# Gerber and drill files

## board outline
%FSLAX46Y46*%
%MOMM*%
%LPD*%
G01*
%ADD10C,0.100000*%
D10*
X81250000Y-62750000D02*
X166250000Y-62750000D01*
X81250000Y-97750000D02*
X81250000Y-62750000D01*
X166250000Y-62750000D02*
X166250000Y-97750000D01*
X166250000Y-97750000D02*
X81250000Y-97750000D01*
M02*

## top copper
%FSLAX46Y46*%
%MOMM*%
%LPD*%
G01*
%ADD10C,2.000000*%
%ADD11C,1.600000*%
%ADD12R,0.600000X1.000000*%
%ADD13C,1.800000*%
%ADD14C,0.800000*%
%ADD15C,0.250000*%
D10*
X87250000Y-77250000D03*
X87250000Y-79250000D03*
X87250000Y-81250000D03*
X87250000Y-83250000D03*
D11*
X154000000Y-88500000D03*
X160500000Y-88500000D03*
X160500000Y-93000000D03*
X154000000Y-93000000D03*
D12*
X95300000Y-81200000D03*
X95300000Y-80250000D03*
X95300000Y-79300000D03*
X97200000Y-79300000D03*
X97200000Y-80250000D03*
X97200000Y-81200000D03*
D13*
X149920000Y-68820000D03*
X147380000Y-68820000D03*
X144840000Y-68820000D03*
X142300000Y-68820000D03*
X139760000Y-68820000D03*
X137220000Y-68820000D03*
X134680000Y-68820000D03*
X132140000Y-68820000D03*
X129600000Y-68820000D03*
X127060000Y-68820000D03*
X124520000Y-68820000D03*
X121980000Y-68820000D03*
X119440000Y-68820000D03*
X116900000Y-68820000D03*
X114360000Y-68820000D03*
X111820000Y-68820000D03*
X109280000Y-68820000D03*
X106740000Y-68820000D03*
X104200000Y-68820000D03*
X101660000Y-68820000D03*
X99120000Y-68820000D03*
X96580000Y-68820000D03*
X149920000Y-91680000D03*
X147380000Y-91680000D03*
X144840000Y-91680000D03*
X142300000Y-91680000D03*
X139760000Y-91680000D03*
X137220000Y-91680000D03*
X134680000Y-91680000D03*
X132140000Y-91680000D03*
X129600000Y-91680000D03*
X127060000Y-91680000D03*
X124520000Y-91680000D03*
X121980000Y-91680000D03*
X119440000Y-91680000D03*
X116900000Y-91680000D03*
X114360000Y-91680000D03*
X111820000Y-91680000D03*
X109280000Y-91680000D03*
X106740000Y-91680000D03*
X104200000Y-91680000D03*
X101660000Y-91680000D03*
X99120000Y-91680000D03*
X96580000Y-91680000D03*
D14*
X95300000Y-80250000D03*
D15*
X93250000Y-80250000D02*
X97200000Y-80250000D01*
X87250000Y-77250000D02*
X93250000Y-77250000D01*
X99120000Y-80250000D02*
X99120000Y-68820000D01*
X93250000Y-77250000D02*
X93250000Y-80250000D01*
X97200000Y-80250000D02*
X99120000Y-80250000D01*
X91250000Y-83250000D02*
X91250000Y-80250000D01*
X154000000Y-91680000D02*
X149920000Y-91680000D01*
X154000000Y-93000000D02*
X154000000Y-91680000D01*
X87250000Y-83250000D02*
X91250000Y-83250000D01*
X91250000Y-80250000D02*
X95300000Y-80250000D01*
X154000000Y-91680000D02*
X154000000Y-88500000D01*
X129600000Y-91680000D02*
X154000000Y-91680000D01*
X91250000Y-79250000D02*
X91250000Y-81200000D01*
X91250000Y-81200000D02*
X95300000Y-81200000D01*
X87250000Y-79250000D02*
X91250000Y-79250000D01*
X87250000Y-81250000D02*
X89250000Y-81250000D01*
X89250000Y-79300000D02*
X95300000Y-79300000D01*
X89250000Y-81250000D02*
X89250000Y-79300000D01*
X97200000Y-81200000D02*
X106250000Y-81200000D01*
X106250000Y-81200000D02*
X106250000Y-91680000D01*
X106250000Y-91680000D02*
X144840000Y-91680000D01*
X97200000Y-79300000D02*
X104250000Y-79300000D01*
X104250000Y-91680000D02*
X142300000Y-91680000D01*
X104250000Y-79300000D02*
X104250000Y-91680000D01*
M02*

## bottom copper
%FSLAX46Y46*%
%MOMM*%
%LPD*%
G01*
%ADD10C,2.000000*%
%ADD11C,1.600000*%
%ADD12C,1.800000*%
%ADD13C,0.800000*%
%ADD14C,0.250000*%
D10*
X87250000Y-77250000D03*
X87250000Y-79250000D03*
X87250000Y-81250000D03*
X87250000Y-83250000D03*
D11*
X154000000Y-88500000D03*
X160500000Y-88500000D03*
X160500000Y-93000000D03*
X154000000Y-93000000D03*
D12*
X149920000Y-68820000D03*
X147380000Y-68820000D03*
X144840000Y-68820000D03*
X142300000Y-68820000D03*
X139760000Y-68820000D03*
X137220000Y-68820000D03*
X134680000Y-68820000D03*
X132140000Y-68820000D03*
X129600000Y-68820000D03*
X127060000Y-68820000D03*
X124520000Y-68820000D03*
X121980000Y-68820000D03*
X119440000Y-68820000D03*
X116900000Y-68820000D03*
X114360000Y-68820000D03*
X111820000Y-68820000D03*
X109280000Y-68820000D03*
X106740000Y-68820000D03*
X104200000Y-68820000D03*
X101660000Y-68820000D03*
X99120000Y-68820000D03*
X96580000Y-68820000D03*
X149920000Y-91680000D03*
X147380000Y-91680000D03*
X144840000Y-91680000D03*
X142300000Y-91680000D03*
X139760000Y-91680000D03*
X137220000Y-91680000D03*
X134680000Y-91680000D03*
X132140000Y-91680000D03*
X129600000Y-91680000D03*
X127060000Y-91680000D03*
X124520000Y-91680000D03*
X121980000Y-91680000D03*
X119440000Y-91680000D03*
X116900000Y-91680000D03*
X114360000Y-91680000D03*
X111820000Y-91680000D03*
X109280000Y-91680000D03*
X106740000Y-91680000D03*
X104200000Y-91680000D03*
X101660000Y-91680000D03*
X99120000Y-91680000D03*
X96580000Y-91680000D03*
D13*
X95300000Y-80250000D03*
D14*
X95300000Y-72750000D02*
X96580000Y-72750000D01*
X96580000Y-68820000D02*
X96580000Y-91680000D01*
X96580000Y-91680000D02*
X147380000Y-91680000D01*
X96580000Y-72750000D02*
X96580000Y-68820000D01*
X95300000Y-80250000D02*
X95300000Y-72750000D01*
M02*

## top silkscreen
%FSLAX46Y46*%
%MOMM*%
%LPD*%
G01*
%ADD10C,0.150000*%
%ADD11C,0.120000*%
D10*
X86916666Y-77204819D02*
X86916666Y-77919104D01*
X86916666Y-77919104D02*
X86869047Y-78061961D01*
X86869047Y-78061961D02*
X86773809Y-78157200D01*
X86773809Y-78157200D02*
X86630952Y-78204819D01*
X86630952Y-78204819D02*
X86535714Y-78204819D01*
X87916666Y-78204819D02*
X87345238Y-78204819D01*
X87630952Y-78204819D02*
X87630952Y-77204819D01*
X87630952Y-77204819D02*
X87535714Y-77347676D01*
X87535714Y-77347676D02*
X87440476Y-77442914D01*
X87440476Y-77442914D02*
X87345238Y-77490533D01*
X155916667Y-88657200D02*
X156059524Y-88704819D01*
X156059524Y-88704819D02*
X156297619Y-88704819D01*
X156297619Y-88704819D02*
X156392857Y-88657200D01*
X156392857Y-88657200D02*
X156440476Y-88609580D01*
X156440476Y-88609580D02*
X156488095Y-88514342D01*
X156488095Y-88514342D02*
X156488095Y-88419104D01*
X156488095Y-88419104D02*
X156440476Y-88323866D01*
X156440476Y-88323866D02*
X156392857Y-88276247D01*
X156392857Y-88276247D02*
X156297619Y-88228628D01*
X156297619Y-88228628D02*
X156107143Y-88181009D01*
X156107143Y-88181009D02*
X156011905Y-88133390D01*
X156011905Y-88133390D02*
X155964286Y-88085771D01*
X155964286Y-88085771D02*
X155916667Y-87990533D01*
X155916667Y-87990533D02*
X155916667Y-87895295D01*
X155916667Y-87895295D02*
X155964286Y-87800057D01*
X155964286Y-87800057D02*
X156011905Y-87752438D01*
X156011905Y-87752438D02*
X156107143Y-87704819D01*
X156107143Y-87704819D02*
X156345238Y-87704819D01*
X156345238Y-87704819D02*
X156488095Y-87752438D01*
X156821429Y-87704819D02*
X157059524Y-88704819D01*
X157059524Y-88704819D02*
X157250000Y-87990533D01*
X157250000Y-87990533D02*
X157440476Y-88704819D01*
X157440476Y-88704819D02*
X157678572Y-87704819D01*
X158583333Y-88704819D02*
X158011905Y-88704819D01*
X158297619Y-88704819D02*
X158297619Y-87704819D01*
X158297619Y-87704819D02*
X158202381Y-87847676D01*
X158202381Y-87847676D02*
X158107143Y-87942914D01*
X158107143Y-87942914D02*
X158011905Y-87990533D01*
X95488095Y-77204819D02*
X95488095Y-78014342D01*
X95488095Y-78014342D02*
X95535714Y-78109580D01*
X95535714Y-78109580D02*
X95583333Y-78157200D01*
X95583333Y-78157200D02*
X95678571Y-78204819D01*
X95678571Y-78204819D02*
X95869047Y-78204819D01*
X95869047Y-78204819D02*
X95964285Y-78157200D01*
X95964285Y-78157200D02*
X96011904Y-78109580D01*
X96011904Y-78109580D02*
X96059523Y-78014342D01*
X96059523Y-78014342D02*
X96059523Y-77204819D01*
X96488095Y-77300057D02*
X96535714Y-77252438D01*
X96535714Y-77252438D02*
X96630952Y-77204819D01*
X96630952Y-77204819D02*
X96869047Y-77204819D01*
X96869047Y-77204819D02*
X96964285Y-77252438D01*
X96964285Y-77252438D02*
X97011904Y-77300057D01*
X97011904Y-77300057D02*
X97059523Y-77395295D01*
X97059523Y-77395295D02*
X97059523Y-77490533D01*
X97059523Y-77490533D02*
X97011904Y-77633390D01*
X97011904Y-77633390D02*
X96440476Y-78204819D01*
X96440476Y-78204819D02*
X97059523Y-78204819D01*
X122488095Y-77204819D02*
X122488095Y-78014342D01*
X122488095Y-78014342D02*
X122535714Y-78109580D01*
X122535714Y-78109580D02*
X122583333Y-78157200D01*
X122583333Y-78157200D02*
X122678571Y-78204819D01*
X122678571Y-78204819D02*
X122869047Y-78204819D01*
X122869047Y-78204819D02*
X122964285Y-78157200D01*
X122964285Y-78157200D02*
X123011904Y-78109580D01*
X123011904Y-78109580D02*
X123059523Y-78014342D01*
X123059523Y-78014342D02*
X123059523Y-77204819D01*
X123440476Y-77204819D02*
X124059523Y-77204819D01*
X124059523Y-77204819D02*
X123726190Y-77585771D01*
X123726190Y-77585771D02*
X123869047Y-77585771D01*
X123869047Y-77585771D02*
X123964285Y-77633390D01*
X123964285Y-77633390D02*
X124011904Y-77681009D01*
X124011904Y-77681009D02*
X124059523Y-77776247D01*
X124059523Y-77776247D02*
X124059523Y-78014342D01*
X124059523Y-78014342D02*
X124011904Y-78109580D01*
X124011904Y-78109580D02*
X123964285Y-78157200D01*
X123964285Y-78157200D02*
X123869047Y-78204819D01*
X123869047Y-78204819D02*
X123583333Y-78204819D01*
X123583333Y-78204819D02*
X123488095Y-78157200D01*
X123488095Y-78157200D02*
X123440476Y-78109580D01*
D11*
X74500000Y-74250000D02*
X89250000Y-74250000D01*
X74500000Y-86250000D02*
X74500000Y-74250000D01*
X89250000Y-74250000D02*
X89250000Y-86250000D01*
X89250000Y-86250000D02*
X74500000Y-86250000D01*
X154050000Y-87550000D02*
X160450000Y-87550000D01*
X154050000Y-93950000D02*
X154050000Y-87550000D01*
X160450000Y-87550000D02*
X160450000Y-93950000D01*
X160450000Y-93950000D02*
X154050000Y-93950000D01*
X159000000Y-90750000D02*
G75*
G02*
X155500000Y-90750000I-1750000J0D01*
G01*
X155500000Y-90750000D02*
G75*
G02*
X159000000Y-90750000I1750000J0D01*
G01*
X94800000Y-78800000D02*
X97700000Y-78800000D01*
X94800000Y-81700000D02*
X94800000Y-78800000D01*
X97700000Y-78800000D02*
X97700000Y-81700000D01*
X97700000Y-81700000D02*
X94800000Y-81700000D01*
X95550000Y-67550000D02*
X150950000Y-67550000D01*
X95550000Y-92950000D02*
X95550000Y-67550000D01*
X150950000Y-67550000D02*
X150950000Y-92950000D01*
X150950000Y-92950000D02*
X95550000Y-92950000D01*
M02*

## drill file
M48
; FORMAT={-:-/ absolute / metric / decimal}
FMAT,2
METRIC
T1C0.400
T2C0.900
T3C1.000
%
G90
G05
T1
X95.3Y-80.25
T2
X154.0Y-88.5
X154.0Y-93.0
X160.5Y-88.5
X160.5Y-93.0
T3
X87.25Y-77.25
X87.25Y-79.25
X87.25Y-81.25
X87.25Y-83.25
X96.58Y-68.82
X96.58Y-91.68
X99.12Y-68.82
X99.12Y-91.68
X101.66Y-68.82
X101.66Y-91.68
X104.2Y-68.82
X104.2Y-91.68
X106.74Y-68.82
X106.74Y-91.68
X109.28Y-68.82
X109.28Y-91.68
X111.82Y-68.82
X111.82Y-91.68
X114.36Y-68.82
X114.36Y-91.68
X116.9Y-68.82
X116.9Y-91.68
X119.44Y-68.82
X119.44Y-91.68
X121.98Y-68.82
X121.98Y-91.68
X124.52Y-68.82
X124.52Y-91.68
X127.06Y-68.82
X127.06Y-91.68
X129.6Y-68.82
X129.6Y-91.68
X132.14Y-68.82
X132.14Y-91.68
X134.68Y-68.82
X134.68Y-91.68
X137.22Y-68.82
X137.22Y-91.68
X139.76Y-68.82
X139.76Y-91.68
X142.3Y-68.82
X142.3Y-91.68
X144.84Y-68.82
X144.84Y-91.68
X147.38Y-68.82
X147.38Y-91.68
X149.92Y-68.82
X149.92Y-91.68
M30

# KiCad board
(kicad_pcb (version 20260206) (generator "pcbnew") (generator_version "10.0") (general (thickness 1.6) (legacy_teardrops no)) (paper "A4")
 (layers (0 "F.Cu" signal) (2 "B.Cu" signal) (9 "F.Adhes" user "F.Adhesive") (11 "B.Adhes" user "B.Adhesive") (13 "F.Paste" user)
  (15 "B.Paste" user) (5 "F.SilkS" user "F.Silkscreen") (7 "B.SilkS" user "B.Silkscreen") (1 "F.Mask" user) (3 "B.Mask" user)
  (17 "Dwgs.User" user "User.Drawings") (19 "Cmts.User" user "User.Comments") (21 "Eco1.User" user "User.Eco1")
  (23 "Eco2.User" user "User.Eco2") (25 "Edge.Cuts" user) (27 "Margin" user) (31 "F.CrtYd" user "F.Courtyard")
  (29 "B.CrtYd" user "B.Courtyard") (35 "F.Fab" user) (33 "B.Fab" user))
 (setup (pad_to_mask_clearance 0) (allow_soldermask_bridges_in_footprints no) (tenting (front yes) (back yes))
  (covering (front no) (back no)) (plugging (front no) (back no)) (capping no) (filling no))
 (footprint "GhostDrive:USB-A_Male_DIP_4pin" (layer "F.Cu") (at 87.25 80.25)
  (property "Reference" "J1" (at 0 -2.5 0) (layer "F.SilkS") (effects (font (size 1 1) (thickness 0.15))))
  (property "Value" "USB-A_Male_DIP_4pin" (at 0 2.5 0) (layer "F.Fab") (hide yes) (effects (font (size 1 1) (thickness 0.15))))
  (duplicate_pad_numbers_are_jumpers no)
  (fp_line (start -12.75 -6) (end 2 -6) (stroke (width 0.12) (type solid)) (layer "F.SilkS"))
  (fp_line (start -12.75 6) (end -12.75 -6) (stroke (width 0.12) (type solid)) (layer "F.SilkS"))
  (fp_line (start 2 -6) (end 2 6) (stroke (width 0.12) (type solid)) (layer "F.SilkS"))
  (fp_line (start 2 6) (end -12.75 6) (stroke (width 0.12) (type solid)) (layer "F.SilkS"))
  (pad "1" thru_hole circle (at 0 -3) (size 2 2) (drill 1) (layers "*.Cu" "*.Mask") (remove_unused_layers no) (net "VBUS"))
  (pad "2" thru_hole circle (at 0 -1) (size 2 2) (drill 1) (layers "*.Cu" "*.Mask") (remove_unused_layers no) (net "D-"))
  (pad "3" thru_hole circle (at 0 1) (size 2 2) (drill 1) (layers "*.Cu" "*.Mask") (remove_unused_layers no) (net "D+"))
  (pad "4" thru_hole circle (at 0 3) (size 2 2) (drill 1) (layers "*.Cu" "*.Mask") (remove_unused_layers no) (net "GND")))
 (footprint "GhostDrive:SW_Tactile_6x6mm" (layer "F.Cu") (at 157.25 90.75)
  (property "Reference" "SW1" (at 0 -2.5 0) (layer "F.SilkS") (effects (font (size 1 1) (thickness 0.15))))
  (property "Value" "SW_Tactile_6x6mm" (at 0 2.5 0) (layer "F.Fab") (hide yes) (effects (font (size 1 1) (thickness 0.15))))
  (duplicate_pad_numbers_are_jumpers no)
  (fp_line (start -3.2 -3.2) (end 3.2 -3.2) (stroke (width 0.12) (type solid)) (layer "F.SilkS"))
  (fp_line (start -3.2 3.2) (end -3.2 -3.2) (stroke (width 0.12) (type solid)) (layer "F.SilkS"))
  (fp_line (start 3.2 -3.2) (end 3.2 3.2) (stroke (width 0.12) (type solid)) (layer "F.SilkS"))
  (fp_line (start 3.2 3.2) (end -3.2 3.2) (stroke (width 0.12) (type solid)) (layer "F.SilkS"))
  (fp_circle (center 0 0) (end 1.75 0) (stroke (width 0.12) (type solid)) (fill no) (layer "F.SilkS"))
  (pad "1" thru_hole circle (at -3.25 -2.25) (size 1.6 1.6) (drill 0.9) (layers "*.Cu" "*.Mask") (remove_unused_layers no) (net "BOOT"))
  (pad "2" thru_hole circle (at 3.25 -2.25) (size 1.6 1.6) (drill 0.9) (layers "*.Cu" "*.Mask") (remove_unused_layers no) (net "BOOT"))
  (pad "3" thru_hole circle (at 3.25 2.25) (size 1.6 1.6) (drill 0.9) (layers "*.Cu" "*.Mask") (remove_unused_layers no) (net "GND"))
  (pad "4" thru_hole circle (at -3.25 2.25) (size 1.6 1.6) (drill 0.9) (layers "*.Cu" "*.Mask") (remove_unused_layers no) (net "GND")))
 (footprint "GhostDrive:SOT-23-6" (layer "F.Cu") (at 96.25 80.25)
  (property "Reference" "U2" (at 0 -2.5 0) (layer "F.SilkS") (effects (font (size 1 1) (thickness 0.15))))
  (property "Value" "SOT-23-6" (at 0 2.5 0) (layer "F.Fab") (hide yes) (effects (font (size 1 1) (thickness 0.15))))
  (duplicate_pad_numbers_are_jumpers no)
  (fp_line (start -1.45 -1.45) (end 1.45 -1.45) (stroke (width 0.12) (type solid)) (layer "F.SilkS"))
  (fp_line (start -1.45 1.45) (end -1.45 -1.45) (stroke (width 0.12) (type solid)) (layer "F.SilkS"))
  (fp_line (start 1.45 -1.45) (end 1.45 1.45) (stroke (width 0.12) (type solid)) (layer "F.SilkS"))
  (fp_line (start 1.45 1.45) (end -1.45 1.45) (stroke (width 0.12) (type solid)) (layer "F.SilkS"))
  (pad "1" smd rect (at -0.95 0.95) (size 0.6 1) (layers "F.Cu" "F.Mask" "F.Paste") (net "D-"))
  (pad "2" smd rect (at -0.95 0) (size 0.6 1) (layers "F.Cu" "F.Mask" "F.Paste") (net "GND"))
  (pad "3" smd rect (at -0.95 -0.95) (size 0.6 1) (layers "F.Cu" "F.Mask" "F.Paste") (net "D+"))
  (pad "4" smd rect (at 0.95 -0.95) (size 0.6 1) (layers "F.Cu" "F.Mask" "F.Paste") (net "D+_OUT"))
  (pad "5" smd rect (at 0.95 0) (size 0.6 1) (layers "F.Cu" "F.Mask" "F.Paste") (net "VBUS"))
  (pad "6" smd rect (at 0.95 0.95) (size 0.6 1) (layers "F.Cu" "F.Mask" "F.Paste") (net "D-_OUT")))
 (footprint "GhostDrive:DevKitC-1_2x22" (layer "F.Cu") (at 123.25 80.25)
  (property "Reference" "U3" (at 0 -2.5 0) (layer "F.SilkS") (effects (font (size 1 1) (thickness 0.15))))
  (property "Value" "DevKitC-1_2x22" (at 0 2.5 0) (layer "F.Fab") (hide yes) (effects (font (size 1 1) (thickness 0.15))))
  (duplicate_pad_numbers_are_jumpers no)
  (fp_line (start -27.7 -12.7) (end 27.7 -12.7) (stroke (width 0.12) (type solid)) (layer "F.SilkS"))
  (fp_line (start -27.7 12.7) (end -27.7 -12.7) (stroke (width 0.12) (type solid)) (layer "F.SilkS"))
  (fp_line (start 27.7 -12.7) (end 27.7 12.7) (stroke (width 0.12) (type solid)) (layer "F.SilkS"))
  (fp_line (start 27.7 12.7) (end -27.7 12.7) (stroke (width 0.12) (type solid)) (layer "F.SilkS"))
  (pad "1" thru_hole circle (at 26.67 -11.43) (size 1.8 1.8) (drill 1) (layers "*.Cu" "*.Mask") (remove_unused_layers no))
  (pad "2" thru_hole circle (at 24.13 -11.43) (size 1.8 1.8) (drill 1) (layers "*.Cu" "*.Mask") (remove_unused_layers no))
  (pad "3" thru_hole circle (at 21.59 -11.43) (size 1.8 1.8) (drill 1) (layers "*.Cu" "*.Mask") (remove_unused_layers no))
  (pad "4" thru_hole circle (at 19.05 -11.43) (size 1.8 1.8) (drill 1) (layers "*.Cu" "*.Mask") (remove_unused_layers no))
  (pad "5" thru_hole circle (at 16.51 -11.43) (size 1.8 1.8) (drill 1) (layers "*.Cu" "*.Mask") (remove_unused_layers no))
  (pad "6" thru_hole circle (at 13.97 -11.43) (size 1.8 1.8) (drill 1) (layers "*.Cu" "*.Mask") (remove_unused_layers no))
  (pad "7" thru_hole circle (at 11.43 -11.43) (size 1.8 1.8) (drill 1) (layers "*.Cu" "*.Mask") (remove_unused_layers no))
  (pad "8" thru_hole circle (at 8.89 -11.43) (size 1.8 1.8) (drill 1) (layers "*.Cu" "*.Mask") (remove_unused_layers no))
  (pad "9" thru_hole circle (at 6.35 -11.43) (size 1.8 1.8) (drill 1) (layers "*.Cu" "*.Mask") (remove_unused_layers no))
  (pad "10" thru_hole circle (at 3.81 -11.43) (size 1.8 1.8) (drill 1) (layers "*.Cu" "*.Mask") (remove_unused_layers no))
  (pad "11" thru_hole circle (at 1.27 -11.43) (size 1.8 1.8) (drill 1) (layers "*.Cu" "*.Mask") (remove_unused_layers no))
  (pad "12" thru_hole circle (at -1.27 -11.43) (size 1.8 1.8) (drill 1) (layers "*.Cu" "*.Mask") (remove_unused_layers no))
  (pad "13" thru_hole circle (at -3.81 -11.43) (size 1.8 1.8) (drill 1) (layers "*.Cu" "*.Mask") (remove_unused_layers no))
  (pad "14" thru_hole circle (at -6.35 -11.43) (size 1.8 1.8) (drill 1) (layers "*.Cu" "*.Mask") (remove_unused_layers no))
  (pad "15" thru_hole circle (at -8.89 -11.43) (size 1.8 1.8) (drill 1) (layers "*.Cu" "*.Mask") (remove_unused_layers no))
  (pad "16" thru_hole circle (at -11.43 -11.43) (size 1.8 1.8) (drill 1) (layers "*.Cu" "*.Mask") (remove_unused_layers no))
  (pad "17" thru_hole circle (at -13.97 -11.43) (size 1.8 1.8) (drill 1) (layers "*.Cu" "*.Mask") (remove_unused_layers no))
  (pad "18" thru_hole circle (at -16.51 -11.43) (size 1.8 1.8) (drill 1) (layers "*.Cu" "*.Mask") (remove_unused_layers no))
  (pad "19" thru_hole circle (at -19.05 -11.43) (size 1.8 1.8) (drill 1) (layers "*.Cu" "*.Mask") (remove_unused_layers no))
  (pad "20" thru_hole circle (at -21.59 -11.43) (size 1.8 1.8) (drill 1) (layers "*.Cu" "*.Mask") (remove_unused_layers no))
  (pad "21" thru_hole circle (at -24.13 -11.43) (size 1.8 1.8) (drill 1) (layers "*.Cu" "*.Mask") (remove_unused_layers no) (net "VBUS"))
  (pad "22" thru_hole circle (at -26.67 -11.43) (size 1.8 1.8) (drill 1) (layers "*.Cu" "*.Mask") (remove_unused_layers no) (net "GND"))
  (pad "23" thru_hole circle (at 26.67 11.43) (size 1.8 1.8) (drill 1) (layers "*.Cu" "*.Mask") (remove_unused_layers no) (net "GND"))
  (pad "24" thru_hole circle (at 24.13 11.43) (size 1.8 1.8) (drill 1) (layers "*.Cu" "*.Mask") (remove_unused_layers no) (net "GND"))
  (pad "25" thru_hole circle (at 21.59 11.43) (size 1.8 1.8) (drill 1) (layers "*.Cu" "*.Mask") (remove_unused_layers no) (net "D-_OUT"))
  (pad "26" thru_hole circle (at 19.05 11.43) (size 1.8 1.8) (drill 1) (layers "*.Cu" "*.Mask") (remove_unused_layers no) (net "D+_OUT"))
  (pad "27" thru_hole circle (at 16.51 11.43) (size 1.8 1.8) (drill 1) (layers "*.Cu" "*.Mask") (remove_unused_layers no))
  (pad "28" thru_hole circle (at 13.97 11.43) (size 1.8 1.8) (drill 1) (layers "*.Cu" "*.Mask") (remove_unused_layers no))
  (pad "29" thru_hole circle (at 11.43 11.43) (size 1.8 1.8) (drill 1) (layers "*.Cu" "*.Mask") (remove_unused_layers no))
  (pad "30" thru_hole circle (at 8.89 11.43) (size 1.8 1.8) (drill 1) (layers "*.Cu" "*.Mask") (remove_unused_layers no))
  (pad "31" thru_hole circle (at 6.35 11.43) (size 1.8 1.8) (drill 1) (layers "*.Cu" "*.Mask") (remove_unused_layers no) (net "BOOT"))
  (pad "32" thru_hole circle (at 3.81 11.43) (size 1.8 1.8) (drill 1) (layers "*.Cu" "*.Mask") (remove_unused_layers no))
  (pad "33" thru_hole circle (at 1.27 11.43) (size 1.8 1.8) (drill 1) (layers "*.Cu" "*.Mask") (remove_unused_layers no))
  (pad "34" thru_hole circle (at -1.27 11.43) (size 1.8 1.8) (drill 1) (layers "*.Cu" "*.Mask") (remove_unused_layers no))
  (pad "35" thru_hole circle (at -3.81 11.43) (size 1.8 1.8) (drill 1) (layers "*.Cu" "*.Mask") (remove_unused_layers no))
  (pad "36" thru_hole circle (at -6.35 11.43) (size 1.8 1.8) (drill 1) (layers "*.Cu" "*.Mask") (remove_unused_layers no))
  (pad "37" thru_hole circle (at -8.89 11.43) (size 1.8 1.8) (drill 1) (layers "*.Cu" "*.Mask") (remove_unused_layers no))
  (pad "38" thru_hole circle (at -11.43 11.43) (size 1.8 1.8) (drill 1) (layers "*.Cu" "*.Mask") (remove_unused_layers no))
  (pad "39" thru_hole circle (at -13.97 11.43) (size 1.8 1.8) (drill 1) (layers "*.Cu" "*.Mask") (remove_unused_layers no))
  (pad "40" thru_hole circle (at -16.51 11.43) (size 1.8 1.8) (drill 1) (layers "*.Cu" "*.Mask") (remove_unused_layers no))
  (pad "41" thru_hole circle (at -19.05 11.43) (size 1.8 1.8) (drill 1) (layers "*.Cu" "*.Mask") (remove_unused_layers no))
  (pad "42" thru_hole circle (at -21.59 11.43) (size 1.8 1.8) (drill 1) (layers "*.Cu" "*.Mask") (remove_unused_layers no))
  (pad "43" thru_hole circle (at -24.13 11.43) (size 1.8 1.8) (drill 1) (layers "*.Cu" "*.Mask") (remove_unused_layers no))
  (pad "44" thru_hole circle (at -26.67 11.43) (size 1.8 1.8) (drill 1) (layers "*.Cu" "*.Mask") (remove_unused_layers no) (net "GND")))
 (gr_line (start 81.25 62.75) (end 166.25 62.75) (stroke (width 0.1) (type solid)) (layer "Edge.Cuts"))
 (gr_line (start 81.25 97.75) (end 81.25 62.75) (stroke (width 0.1) (type solid)) (layer "Edge.Cuts"))
 (gr_line (start 166.25 62.75) (end 166.25 97.75) (stroke (width 0.1) (type solid)) (layer "Edge.Cuts"))
 (gr_line (start 166.25 97.75) (end 81.25 97.75) (stroke (width 0.1) (type solid)) (layer "Edge.Cuts"))
 (segment (start 93.25 80.25) (end 97.2 80.25) (width 0.25) (layer "F.Cu") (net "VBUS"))
 (segment (start 87.25 77.25) (end 93.25 77.25) (width 0.25) (layer "F.Cu") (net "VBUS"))
 (segment (start 99.12 80.25) (end 99.12 68.82) (width 0.25) (layer "F.Cu") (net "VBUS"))
 (segment (start 93.25 77.25) (end 93.25 80.25) (width 0.25) (layer "F.Cu") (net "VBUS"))
 (segment (start 97.2 80.25) (end 99.12 80.25) (width 0.25) (layer "F.Cu") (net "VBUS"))
 (segment (start 91.25 83.25) (end 91.25 80.25) (width 0.25) (layer "F.Cu") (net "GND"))
 (segment (start 154 91.68) (end 149.92 91.68) (width 0.25) (layer "F.Cu") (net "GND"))
 (segment (start 154 93) (end 154 91.68) (width 0.25) (layer "F.Cu") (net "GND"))
 (segment (start 87.25 83.25) (end 91.25 83.25) (width 0.25) (layer "F.Cu") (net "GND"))
 (segment (start 91.25 80.25) (end 95.3 80.25) (width 0.25) (layer "F.Cu") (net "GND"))
 (via (at 95.3 80.25) (size 0.8) (drill 0.4) (layers "F.Cu" "B.Cu") (capping no) (covering (front no) (back no))
  (plugging (front no) (back no)) (filling no) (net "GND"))
 (segment (start 95.3 72.75) (end 96.58 72.75) (width 0.25) (layer "B.Cu") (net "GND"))
 (segment (start 96.58 68.82) (end 96.58 91.68) (width 0.25) (layer "B.Cu") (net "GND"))
 (segment (start 96.58 91.68) (end 147.38 91.68) (width 0.25) (layer "B.Cu") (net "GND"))
 (segment (start 96.58 72.75) (end 96.58 68.82) (width 0.25) (layer "B.Cu") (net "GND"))
 (segment (start 95.3 80.25) (end 95.3 72.75) (width 0.25) (layer "B.Cu") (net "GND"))
 (segment (start 154 91.68) (end 154 88.5) (width 0.25) (layer "F.Cu") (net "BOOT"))
 (segment (start 129.6 91.68) (end 154 91.68) (width 0.25) (layer "F.Cu") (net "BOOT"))
 (segment (start 91.25 79.25) (end 91.25 81.2) (width 0.25) (layer "F.Cu") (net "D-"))
 (segment (start 91.25 81.2) (end 95.3 81.2) (width 0.25) (layer "F.Cu") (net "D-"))
 (segment (start 87.25 79.25) (end 91.25 79.25) (width 0.25) (layer "F.Cu") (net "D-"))
 (segment (start 87.25 81.25) (end 89.25 81.25) (width 0.25) (layer "F.Cu") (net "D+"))
 (segment (start 89.25 79.3) (end 95.3 79.3) (width 0.25) (layer "F.Cu") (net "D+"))
 (segment (start 89.25 81.25) (end 89.25 79.3) (width 0.25) (layer "F.Cu") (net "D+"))
 (segment (start 97.2 81.2) (end 106.25 81.2) (width 0.25) (layer "F.Cu") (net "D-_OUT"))
 (segment (start 106.25 81.2) (end 106.25 91.68) (width 0.25) (layer "F.Cu") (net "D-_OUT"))
 (segment (start 106.25 91.68) (end 144.84 91.68) (width 0.25) (layer "F.Cu") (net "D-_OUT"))
 (segment (start 97.2 79.3) (end 104.25 79.3) (width 0.25) (layer "F.Cu") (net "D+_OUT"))
 (segment (start 104.25 91.68) (end 142.3 91.68) (width 0.25) (layer "F.Cu") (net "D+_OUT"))
 (segment (start 104.25 79.3) (end 104.25 91.68) (width 0.25) (layer "F.Cu") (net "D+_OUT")))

